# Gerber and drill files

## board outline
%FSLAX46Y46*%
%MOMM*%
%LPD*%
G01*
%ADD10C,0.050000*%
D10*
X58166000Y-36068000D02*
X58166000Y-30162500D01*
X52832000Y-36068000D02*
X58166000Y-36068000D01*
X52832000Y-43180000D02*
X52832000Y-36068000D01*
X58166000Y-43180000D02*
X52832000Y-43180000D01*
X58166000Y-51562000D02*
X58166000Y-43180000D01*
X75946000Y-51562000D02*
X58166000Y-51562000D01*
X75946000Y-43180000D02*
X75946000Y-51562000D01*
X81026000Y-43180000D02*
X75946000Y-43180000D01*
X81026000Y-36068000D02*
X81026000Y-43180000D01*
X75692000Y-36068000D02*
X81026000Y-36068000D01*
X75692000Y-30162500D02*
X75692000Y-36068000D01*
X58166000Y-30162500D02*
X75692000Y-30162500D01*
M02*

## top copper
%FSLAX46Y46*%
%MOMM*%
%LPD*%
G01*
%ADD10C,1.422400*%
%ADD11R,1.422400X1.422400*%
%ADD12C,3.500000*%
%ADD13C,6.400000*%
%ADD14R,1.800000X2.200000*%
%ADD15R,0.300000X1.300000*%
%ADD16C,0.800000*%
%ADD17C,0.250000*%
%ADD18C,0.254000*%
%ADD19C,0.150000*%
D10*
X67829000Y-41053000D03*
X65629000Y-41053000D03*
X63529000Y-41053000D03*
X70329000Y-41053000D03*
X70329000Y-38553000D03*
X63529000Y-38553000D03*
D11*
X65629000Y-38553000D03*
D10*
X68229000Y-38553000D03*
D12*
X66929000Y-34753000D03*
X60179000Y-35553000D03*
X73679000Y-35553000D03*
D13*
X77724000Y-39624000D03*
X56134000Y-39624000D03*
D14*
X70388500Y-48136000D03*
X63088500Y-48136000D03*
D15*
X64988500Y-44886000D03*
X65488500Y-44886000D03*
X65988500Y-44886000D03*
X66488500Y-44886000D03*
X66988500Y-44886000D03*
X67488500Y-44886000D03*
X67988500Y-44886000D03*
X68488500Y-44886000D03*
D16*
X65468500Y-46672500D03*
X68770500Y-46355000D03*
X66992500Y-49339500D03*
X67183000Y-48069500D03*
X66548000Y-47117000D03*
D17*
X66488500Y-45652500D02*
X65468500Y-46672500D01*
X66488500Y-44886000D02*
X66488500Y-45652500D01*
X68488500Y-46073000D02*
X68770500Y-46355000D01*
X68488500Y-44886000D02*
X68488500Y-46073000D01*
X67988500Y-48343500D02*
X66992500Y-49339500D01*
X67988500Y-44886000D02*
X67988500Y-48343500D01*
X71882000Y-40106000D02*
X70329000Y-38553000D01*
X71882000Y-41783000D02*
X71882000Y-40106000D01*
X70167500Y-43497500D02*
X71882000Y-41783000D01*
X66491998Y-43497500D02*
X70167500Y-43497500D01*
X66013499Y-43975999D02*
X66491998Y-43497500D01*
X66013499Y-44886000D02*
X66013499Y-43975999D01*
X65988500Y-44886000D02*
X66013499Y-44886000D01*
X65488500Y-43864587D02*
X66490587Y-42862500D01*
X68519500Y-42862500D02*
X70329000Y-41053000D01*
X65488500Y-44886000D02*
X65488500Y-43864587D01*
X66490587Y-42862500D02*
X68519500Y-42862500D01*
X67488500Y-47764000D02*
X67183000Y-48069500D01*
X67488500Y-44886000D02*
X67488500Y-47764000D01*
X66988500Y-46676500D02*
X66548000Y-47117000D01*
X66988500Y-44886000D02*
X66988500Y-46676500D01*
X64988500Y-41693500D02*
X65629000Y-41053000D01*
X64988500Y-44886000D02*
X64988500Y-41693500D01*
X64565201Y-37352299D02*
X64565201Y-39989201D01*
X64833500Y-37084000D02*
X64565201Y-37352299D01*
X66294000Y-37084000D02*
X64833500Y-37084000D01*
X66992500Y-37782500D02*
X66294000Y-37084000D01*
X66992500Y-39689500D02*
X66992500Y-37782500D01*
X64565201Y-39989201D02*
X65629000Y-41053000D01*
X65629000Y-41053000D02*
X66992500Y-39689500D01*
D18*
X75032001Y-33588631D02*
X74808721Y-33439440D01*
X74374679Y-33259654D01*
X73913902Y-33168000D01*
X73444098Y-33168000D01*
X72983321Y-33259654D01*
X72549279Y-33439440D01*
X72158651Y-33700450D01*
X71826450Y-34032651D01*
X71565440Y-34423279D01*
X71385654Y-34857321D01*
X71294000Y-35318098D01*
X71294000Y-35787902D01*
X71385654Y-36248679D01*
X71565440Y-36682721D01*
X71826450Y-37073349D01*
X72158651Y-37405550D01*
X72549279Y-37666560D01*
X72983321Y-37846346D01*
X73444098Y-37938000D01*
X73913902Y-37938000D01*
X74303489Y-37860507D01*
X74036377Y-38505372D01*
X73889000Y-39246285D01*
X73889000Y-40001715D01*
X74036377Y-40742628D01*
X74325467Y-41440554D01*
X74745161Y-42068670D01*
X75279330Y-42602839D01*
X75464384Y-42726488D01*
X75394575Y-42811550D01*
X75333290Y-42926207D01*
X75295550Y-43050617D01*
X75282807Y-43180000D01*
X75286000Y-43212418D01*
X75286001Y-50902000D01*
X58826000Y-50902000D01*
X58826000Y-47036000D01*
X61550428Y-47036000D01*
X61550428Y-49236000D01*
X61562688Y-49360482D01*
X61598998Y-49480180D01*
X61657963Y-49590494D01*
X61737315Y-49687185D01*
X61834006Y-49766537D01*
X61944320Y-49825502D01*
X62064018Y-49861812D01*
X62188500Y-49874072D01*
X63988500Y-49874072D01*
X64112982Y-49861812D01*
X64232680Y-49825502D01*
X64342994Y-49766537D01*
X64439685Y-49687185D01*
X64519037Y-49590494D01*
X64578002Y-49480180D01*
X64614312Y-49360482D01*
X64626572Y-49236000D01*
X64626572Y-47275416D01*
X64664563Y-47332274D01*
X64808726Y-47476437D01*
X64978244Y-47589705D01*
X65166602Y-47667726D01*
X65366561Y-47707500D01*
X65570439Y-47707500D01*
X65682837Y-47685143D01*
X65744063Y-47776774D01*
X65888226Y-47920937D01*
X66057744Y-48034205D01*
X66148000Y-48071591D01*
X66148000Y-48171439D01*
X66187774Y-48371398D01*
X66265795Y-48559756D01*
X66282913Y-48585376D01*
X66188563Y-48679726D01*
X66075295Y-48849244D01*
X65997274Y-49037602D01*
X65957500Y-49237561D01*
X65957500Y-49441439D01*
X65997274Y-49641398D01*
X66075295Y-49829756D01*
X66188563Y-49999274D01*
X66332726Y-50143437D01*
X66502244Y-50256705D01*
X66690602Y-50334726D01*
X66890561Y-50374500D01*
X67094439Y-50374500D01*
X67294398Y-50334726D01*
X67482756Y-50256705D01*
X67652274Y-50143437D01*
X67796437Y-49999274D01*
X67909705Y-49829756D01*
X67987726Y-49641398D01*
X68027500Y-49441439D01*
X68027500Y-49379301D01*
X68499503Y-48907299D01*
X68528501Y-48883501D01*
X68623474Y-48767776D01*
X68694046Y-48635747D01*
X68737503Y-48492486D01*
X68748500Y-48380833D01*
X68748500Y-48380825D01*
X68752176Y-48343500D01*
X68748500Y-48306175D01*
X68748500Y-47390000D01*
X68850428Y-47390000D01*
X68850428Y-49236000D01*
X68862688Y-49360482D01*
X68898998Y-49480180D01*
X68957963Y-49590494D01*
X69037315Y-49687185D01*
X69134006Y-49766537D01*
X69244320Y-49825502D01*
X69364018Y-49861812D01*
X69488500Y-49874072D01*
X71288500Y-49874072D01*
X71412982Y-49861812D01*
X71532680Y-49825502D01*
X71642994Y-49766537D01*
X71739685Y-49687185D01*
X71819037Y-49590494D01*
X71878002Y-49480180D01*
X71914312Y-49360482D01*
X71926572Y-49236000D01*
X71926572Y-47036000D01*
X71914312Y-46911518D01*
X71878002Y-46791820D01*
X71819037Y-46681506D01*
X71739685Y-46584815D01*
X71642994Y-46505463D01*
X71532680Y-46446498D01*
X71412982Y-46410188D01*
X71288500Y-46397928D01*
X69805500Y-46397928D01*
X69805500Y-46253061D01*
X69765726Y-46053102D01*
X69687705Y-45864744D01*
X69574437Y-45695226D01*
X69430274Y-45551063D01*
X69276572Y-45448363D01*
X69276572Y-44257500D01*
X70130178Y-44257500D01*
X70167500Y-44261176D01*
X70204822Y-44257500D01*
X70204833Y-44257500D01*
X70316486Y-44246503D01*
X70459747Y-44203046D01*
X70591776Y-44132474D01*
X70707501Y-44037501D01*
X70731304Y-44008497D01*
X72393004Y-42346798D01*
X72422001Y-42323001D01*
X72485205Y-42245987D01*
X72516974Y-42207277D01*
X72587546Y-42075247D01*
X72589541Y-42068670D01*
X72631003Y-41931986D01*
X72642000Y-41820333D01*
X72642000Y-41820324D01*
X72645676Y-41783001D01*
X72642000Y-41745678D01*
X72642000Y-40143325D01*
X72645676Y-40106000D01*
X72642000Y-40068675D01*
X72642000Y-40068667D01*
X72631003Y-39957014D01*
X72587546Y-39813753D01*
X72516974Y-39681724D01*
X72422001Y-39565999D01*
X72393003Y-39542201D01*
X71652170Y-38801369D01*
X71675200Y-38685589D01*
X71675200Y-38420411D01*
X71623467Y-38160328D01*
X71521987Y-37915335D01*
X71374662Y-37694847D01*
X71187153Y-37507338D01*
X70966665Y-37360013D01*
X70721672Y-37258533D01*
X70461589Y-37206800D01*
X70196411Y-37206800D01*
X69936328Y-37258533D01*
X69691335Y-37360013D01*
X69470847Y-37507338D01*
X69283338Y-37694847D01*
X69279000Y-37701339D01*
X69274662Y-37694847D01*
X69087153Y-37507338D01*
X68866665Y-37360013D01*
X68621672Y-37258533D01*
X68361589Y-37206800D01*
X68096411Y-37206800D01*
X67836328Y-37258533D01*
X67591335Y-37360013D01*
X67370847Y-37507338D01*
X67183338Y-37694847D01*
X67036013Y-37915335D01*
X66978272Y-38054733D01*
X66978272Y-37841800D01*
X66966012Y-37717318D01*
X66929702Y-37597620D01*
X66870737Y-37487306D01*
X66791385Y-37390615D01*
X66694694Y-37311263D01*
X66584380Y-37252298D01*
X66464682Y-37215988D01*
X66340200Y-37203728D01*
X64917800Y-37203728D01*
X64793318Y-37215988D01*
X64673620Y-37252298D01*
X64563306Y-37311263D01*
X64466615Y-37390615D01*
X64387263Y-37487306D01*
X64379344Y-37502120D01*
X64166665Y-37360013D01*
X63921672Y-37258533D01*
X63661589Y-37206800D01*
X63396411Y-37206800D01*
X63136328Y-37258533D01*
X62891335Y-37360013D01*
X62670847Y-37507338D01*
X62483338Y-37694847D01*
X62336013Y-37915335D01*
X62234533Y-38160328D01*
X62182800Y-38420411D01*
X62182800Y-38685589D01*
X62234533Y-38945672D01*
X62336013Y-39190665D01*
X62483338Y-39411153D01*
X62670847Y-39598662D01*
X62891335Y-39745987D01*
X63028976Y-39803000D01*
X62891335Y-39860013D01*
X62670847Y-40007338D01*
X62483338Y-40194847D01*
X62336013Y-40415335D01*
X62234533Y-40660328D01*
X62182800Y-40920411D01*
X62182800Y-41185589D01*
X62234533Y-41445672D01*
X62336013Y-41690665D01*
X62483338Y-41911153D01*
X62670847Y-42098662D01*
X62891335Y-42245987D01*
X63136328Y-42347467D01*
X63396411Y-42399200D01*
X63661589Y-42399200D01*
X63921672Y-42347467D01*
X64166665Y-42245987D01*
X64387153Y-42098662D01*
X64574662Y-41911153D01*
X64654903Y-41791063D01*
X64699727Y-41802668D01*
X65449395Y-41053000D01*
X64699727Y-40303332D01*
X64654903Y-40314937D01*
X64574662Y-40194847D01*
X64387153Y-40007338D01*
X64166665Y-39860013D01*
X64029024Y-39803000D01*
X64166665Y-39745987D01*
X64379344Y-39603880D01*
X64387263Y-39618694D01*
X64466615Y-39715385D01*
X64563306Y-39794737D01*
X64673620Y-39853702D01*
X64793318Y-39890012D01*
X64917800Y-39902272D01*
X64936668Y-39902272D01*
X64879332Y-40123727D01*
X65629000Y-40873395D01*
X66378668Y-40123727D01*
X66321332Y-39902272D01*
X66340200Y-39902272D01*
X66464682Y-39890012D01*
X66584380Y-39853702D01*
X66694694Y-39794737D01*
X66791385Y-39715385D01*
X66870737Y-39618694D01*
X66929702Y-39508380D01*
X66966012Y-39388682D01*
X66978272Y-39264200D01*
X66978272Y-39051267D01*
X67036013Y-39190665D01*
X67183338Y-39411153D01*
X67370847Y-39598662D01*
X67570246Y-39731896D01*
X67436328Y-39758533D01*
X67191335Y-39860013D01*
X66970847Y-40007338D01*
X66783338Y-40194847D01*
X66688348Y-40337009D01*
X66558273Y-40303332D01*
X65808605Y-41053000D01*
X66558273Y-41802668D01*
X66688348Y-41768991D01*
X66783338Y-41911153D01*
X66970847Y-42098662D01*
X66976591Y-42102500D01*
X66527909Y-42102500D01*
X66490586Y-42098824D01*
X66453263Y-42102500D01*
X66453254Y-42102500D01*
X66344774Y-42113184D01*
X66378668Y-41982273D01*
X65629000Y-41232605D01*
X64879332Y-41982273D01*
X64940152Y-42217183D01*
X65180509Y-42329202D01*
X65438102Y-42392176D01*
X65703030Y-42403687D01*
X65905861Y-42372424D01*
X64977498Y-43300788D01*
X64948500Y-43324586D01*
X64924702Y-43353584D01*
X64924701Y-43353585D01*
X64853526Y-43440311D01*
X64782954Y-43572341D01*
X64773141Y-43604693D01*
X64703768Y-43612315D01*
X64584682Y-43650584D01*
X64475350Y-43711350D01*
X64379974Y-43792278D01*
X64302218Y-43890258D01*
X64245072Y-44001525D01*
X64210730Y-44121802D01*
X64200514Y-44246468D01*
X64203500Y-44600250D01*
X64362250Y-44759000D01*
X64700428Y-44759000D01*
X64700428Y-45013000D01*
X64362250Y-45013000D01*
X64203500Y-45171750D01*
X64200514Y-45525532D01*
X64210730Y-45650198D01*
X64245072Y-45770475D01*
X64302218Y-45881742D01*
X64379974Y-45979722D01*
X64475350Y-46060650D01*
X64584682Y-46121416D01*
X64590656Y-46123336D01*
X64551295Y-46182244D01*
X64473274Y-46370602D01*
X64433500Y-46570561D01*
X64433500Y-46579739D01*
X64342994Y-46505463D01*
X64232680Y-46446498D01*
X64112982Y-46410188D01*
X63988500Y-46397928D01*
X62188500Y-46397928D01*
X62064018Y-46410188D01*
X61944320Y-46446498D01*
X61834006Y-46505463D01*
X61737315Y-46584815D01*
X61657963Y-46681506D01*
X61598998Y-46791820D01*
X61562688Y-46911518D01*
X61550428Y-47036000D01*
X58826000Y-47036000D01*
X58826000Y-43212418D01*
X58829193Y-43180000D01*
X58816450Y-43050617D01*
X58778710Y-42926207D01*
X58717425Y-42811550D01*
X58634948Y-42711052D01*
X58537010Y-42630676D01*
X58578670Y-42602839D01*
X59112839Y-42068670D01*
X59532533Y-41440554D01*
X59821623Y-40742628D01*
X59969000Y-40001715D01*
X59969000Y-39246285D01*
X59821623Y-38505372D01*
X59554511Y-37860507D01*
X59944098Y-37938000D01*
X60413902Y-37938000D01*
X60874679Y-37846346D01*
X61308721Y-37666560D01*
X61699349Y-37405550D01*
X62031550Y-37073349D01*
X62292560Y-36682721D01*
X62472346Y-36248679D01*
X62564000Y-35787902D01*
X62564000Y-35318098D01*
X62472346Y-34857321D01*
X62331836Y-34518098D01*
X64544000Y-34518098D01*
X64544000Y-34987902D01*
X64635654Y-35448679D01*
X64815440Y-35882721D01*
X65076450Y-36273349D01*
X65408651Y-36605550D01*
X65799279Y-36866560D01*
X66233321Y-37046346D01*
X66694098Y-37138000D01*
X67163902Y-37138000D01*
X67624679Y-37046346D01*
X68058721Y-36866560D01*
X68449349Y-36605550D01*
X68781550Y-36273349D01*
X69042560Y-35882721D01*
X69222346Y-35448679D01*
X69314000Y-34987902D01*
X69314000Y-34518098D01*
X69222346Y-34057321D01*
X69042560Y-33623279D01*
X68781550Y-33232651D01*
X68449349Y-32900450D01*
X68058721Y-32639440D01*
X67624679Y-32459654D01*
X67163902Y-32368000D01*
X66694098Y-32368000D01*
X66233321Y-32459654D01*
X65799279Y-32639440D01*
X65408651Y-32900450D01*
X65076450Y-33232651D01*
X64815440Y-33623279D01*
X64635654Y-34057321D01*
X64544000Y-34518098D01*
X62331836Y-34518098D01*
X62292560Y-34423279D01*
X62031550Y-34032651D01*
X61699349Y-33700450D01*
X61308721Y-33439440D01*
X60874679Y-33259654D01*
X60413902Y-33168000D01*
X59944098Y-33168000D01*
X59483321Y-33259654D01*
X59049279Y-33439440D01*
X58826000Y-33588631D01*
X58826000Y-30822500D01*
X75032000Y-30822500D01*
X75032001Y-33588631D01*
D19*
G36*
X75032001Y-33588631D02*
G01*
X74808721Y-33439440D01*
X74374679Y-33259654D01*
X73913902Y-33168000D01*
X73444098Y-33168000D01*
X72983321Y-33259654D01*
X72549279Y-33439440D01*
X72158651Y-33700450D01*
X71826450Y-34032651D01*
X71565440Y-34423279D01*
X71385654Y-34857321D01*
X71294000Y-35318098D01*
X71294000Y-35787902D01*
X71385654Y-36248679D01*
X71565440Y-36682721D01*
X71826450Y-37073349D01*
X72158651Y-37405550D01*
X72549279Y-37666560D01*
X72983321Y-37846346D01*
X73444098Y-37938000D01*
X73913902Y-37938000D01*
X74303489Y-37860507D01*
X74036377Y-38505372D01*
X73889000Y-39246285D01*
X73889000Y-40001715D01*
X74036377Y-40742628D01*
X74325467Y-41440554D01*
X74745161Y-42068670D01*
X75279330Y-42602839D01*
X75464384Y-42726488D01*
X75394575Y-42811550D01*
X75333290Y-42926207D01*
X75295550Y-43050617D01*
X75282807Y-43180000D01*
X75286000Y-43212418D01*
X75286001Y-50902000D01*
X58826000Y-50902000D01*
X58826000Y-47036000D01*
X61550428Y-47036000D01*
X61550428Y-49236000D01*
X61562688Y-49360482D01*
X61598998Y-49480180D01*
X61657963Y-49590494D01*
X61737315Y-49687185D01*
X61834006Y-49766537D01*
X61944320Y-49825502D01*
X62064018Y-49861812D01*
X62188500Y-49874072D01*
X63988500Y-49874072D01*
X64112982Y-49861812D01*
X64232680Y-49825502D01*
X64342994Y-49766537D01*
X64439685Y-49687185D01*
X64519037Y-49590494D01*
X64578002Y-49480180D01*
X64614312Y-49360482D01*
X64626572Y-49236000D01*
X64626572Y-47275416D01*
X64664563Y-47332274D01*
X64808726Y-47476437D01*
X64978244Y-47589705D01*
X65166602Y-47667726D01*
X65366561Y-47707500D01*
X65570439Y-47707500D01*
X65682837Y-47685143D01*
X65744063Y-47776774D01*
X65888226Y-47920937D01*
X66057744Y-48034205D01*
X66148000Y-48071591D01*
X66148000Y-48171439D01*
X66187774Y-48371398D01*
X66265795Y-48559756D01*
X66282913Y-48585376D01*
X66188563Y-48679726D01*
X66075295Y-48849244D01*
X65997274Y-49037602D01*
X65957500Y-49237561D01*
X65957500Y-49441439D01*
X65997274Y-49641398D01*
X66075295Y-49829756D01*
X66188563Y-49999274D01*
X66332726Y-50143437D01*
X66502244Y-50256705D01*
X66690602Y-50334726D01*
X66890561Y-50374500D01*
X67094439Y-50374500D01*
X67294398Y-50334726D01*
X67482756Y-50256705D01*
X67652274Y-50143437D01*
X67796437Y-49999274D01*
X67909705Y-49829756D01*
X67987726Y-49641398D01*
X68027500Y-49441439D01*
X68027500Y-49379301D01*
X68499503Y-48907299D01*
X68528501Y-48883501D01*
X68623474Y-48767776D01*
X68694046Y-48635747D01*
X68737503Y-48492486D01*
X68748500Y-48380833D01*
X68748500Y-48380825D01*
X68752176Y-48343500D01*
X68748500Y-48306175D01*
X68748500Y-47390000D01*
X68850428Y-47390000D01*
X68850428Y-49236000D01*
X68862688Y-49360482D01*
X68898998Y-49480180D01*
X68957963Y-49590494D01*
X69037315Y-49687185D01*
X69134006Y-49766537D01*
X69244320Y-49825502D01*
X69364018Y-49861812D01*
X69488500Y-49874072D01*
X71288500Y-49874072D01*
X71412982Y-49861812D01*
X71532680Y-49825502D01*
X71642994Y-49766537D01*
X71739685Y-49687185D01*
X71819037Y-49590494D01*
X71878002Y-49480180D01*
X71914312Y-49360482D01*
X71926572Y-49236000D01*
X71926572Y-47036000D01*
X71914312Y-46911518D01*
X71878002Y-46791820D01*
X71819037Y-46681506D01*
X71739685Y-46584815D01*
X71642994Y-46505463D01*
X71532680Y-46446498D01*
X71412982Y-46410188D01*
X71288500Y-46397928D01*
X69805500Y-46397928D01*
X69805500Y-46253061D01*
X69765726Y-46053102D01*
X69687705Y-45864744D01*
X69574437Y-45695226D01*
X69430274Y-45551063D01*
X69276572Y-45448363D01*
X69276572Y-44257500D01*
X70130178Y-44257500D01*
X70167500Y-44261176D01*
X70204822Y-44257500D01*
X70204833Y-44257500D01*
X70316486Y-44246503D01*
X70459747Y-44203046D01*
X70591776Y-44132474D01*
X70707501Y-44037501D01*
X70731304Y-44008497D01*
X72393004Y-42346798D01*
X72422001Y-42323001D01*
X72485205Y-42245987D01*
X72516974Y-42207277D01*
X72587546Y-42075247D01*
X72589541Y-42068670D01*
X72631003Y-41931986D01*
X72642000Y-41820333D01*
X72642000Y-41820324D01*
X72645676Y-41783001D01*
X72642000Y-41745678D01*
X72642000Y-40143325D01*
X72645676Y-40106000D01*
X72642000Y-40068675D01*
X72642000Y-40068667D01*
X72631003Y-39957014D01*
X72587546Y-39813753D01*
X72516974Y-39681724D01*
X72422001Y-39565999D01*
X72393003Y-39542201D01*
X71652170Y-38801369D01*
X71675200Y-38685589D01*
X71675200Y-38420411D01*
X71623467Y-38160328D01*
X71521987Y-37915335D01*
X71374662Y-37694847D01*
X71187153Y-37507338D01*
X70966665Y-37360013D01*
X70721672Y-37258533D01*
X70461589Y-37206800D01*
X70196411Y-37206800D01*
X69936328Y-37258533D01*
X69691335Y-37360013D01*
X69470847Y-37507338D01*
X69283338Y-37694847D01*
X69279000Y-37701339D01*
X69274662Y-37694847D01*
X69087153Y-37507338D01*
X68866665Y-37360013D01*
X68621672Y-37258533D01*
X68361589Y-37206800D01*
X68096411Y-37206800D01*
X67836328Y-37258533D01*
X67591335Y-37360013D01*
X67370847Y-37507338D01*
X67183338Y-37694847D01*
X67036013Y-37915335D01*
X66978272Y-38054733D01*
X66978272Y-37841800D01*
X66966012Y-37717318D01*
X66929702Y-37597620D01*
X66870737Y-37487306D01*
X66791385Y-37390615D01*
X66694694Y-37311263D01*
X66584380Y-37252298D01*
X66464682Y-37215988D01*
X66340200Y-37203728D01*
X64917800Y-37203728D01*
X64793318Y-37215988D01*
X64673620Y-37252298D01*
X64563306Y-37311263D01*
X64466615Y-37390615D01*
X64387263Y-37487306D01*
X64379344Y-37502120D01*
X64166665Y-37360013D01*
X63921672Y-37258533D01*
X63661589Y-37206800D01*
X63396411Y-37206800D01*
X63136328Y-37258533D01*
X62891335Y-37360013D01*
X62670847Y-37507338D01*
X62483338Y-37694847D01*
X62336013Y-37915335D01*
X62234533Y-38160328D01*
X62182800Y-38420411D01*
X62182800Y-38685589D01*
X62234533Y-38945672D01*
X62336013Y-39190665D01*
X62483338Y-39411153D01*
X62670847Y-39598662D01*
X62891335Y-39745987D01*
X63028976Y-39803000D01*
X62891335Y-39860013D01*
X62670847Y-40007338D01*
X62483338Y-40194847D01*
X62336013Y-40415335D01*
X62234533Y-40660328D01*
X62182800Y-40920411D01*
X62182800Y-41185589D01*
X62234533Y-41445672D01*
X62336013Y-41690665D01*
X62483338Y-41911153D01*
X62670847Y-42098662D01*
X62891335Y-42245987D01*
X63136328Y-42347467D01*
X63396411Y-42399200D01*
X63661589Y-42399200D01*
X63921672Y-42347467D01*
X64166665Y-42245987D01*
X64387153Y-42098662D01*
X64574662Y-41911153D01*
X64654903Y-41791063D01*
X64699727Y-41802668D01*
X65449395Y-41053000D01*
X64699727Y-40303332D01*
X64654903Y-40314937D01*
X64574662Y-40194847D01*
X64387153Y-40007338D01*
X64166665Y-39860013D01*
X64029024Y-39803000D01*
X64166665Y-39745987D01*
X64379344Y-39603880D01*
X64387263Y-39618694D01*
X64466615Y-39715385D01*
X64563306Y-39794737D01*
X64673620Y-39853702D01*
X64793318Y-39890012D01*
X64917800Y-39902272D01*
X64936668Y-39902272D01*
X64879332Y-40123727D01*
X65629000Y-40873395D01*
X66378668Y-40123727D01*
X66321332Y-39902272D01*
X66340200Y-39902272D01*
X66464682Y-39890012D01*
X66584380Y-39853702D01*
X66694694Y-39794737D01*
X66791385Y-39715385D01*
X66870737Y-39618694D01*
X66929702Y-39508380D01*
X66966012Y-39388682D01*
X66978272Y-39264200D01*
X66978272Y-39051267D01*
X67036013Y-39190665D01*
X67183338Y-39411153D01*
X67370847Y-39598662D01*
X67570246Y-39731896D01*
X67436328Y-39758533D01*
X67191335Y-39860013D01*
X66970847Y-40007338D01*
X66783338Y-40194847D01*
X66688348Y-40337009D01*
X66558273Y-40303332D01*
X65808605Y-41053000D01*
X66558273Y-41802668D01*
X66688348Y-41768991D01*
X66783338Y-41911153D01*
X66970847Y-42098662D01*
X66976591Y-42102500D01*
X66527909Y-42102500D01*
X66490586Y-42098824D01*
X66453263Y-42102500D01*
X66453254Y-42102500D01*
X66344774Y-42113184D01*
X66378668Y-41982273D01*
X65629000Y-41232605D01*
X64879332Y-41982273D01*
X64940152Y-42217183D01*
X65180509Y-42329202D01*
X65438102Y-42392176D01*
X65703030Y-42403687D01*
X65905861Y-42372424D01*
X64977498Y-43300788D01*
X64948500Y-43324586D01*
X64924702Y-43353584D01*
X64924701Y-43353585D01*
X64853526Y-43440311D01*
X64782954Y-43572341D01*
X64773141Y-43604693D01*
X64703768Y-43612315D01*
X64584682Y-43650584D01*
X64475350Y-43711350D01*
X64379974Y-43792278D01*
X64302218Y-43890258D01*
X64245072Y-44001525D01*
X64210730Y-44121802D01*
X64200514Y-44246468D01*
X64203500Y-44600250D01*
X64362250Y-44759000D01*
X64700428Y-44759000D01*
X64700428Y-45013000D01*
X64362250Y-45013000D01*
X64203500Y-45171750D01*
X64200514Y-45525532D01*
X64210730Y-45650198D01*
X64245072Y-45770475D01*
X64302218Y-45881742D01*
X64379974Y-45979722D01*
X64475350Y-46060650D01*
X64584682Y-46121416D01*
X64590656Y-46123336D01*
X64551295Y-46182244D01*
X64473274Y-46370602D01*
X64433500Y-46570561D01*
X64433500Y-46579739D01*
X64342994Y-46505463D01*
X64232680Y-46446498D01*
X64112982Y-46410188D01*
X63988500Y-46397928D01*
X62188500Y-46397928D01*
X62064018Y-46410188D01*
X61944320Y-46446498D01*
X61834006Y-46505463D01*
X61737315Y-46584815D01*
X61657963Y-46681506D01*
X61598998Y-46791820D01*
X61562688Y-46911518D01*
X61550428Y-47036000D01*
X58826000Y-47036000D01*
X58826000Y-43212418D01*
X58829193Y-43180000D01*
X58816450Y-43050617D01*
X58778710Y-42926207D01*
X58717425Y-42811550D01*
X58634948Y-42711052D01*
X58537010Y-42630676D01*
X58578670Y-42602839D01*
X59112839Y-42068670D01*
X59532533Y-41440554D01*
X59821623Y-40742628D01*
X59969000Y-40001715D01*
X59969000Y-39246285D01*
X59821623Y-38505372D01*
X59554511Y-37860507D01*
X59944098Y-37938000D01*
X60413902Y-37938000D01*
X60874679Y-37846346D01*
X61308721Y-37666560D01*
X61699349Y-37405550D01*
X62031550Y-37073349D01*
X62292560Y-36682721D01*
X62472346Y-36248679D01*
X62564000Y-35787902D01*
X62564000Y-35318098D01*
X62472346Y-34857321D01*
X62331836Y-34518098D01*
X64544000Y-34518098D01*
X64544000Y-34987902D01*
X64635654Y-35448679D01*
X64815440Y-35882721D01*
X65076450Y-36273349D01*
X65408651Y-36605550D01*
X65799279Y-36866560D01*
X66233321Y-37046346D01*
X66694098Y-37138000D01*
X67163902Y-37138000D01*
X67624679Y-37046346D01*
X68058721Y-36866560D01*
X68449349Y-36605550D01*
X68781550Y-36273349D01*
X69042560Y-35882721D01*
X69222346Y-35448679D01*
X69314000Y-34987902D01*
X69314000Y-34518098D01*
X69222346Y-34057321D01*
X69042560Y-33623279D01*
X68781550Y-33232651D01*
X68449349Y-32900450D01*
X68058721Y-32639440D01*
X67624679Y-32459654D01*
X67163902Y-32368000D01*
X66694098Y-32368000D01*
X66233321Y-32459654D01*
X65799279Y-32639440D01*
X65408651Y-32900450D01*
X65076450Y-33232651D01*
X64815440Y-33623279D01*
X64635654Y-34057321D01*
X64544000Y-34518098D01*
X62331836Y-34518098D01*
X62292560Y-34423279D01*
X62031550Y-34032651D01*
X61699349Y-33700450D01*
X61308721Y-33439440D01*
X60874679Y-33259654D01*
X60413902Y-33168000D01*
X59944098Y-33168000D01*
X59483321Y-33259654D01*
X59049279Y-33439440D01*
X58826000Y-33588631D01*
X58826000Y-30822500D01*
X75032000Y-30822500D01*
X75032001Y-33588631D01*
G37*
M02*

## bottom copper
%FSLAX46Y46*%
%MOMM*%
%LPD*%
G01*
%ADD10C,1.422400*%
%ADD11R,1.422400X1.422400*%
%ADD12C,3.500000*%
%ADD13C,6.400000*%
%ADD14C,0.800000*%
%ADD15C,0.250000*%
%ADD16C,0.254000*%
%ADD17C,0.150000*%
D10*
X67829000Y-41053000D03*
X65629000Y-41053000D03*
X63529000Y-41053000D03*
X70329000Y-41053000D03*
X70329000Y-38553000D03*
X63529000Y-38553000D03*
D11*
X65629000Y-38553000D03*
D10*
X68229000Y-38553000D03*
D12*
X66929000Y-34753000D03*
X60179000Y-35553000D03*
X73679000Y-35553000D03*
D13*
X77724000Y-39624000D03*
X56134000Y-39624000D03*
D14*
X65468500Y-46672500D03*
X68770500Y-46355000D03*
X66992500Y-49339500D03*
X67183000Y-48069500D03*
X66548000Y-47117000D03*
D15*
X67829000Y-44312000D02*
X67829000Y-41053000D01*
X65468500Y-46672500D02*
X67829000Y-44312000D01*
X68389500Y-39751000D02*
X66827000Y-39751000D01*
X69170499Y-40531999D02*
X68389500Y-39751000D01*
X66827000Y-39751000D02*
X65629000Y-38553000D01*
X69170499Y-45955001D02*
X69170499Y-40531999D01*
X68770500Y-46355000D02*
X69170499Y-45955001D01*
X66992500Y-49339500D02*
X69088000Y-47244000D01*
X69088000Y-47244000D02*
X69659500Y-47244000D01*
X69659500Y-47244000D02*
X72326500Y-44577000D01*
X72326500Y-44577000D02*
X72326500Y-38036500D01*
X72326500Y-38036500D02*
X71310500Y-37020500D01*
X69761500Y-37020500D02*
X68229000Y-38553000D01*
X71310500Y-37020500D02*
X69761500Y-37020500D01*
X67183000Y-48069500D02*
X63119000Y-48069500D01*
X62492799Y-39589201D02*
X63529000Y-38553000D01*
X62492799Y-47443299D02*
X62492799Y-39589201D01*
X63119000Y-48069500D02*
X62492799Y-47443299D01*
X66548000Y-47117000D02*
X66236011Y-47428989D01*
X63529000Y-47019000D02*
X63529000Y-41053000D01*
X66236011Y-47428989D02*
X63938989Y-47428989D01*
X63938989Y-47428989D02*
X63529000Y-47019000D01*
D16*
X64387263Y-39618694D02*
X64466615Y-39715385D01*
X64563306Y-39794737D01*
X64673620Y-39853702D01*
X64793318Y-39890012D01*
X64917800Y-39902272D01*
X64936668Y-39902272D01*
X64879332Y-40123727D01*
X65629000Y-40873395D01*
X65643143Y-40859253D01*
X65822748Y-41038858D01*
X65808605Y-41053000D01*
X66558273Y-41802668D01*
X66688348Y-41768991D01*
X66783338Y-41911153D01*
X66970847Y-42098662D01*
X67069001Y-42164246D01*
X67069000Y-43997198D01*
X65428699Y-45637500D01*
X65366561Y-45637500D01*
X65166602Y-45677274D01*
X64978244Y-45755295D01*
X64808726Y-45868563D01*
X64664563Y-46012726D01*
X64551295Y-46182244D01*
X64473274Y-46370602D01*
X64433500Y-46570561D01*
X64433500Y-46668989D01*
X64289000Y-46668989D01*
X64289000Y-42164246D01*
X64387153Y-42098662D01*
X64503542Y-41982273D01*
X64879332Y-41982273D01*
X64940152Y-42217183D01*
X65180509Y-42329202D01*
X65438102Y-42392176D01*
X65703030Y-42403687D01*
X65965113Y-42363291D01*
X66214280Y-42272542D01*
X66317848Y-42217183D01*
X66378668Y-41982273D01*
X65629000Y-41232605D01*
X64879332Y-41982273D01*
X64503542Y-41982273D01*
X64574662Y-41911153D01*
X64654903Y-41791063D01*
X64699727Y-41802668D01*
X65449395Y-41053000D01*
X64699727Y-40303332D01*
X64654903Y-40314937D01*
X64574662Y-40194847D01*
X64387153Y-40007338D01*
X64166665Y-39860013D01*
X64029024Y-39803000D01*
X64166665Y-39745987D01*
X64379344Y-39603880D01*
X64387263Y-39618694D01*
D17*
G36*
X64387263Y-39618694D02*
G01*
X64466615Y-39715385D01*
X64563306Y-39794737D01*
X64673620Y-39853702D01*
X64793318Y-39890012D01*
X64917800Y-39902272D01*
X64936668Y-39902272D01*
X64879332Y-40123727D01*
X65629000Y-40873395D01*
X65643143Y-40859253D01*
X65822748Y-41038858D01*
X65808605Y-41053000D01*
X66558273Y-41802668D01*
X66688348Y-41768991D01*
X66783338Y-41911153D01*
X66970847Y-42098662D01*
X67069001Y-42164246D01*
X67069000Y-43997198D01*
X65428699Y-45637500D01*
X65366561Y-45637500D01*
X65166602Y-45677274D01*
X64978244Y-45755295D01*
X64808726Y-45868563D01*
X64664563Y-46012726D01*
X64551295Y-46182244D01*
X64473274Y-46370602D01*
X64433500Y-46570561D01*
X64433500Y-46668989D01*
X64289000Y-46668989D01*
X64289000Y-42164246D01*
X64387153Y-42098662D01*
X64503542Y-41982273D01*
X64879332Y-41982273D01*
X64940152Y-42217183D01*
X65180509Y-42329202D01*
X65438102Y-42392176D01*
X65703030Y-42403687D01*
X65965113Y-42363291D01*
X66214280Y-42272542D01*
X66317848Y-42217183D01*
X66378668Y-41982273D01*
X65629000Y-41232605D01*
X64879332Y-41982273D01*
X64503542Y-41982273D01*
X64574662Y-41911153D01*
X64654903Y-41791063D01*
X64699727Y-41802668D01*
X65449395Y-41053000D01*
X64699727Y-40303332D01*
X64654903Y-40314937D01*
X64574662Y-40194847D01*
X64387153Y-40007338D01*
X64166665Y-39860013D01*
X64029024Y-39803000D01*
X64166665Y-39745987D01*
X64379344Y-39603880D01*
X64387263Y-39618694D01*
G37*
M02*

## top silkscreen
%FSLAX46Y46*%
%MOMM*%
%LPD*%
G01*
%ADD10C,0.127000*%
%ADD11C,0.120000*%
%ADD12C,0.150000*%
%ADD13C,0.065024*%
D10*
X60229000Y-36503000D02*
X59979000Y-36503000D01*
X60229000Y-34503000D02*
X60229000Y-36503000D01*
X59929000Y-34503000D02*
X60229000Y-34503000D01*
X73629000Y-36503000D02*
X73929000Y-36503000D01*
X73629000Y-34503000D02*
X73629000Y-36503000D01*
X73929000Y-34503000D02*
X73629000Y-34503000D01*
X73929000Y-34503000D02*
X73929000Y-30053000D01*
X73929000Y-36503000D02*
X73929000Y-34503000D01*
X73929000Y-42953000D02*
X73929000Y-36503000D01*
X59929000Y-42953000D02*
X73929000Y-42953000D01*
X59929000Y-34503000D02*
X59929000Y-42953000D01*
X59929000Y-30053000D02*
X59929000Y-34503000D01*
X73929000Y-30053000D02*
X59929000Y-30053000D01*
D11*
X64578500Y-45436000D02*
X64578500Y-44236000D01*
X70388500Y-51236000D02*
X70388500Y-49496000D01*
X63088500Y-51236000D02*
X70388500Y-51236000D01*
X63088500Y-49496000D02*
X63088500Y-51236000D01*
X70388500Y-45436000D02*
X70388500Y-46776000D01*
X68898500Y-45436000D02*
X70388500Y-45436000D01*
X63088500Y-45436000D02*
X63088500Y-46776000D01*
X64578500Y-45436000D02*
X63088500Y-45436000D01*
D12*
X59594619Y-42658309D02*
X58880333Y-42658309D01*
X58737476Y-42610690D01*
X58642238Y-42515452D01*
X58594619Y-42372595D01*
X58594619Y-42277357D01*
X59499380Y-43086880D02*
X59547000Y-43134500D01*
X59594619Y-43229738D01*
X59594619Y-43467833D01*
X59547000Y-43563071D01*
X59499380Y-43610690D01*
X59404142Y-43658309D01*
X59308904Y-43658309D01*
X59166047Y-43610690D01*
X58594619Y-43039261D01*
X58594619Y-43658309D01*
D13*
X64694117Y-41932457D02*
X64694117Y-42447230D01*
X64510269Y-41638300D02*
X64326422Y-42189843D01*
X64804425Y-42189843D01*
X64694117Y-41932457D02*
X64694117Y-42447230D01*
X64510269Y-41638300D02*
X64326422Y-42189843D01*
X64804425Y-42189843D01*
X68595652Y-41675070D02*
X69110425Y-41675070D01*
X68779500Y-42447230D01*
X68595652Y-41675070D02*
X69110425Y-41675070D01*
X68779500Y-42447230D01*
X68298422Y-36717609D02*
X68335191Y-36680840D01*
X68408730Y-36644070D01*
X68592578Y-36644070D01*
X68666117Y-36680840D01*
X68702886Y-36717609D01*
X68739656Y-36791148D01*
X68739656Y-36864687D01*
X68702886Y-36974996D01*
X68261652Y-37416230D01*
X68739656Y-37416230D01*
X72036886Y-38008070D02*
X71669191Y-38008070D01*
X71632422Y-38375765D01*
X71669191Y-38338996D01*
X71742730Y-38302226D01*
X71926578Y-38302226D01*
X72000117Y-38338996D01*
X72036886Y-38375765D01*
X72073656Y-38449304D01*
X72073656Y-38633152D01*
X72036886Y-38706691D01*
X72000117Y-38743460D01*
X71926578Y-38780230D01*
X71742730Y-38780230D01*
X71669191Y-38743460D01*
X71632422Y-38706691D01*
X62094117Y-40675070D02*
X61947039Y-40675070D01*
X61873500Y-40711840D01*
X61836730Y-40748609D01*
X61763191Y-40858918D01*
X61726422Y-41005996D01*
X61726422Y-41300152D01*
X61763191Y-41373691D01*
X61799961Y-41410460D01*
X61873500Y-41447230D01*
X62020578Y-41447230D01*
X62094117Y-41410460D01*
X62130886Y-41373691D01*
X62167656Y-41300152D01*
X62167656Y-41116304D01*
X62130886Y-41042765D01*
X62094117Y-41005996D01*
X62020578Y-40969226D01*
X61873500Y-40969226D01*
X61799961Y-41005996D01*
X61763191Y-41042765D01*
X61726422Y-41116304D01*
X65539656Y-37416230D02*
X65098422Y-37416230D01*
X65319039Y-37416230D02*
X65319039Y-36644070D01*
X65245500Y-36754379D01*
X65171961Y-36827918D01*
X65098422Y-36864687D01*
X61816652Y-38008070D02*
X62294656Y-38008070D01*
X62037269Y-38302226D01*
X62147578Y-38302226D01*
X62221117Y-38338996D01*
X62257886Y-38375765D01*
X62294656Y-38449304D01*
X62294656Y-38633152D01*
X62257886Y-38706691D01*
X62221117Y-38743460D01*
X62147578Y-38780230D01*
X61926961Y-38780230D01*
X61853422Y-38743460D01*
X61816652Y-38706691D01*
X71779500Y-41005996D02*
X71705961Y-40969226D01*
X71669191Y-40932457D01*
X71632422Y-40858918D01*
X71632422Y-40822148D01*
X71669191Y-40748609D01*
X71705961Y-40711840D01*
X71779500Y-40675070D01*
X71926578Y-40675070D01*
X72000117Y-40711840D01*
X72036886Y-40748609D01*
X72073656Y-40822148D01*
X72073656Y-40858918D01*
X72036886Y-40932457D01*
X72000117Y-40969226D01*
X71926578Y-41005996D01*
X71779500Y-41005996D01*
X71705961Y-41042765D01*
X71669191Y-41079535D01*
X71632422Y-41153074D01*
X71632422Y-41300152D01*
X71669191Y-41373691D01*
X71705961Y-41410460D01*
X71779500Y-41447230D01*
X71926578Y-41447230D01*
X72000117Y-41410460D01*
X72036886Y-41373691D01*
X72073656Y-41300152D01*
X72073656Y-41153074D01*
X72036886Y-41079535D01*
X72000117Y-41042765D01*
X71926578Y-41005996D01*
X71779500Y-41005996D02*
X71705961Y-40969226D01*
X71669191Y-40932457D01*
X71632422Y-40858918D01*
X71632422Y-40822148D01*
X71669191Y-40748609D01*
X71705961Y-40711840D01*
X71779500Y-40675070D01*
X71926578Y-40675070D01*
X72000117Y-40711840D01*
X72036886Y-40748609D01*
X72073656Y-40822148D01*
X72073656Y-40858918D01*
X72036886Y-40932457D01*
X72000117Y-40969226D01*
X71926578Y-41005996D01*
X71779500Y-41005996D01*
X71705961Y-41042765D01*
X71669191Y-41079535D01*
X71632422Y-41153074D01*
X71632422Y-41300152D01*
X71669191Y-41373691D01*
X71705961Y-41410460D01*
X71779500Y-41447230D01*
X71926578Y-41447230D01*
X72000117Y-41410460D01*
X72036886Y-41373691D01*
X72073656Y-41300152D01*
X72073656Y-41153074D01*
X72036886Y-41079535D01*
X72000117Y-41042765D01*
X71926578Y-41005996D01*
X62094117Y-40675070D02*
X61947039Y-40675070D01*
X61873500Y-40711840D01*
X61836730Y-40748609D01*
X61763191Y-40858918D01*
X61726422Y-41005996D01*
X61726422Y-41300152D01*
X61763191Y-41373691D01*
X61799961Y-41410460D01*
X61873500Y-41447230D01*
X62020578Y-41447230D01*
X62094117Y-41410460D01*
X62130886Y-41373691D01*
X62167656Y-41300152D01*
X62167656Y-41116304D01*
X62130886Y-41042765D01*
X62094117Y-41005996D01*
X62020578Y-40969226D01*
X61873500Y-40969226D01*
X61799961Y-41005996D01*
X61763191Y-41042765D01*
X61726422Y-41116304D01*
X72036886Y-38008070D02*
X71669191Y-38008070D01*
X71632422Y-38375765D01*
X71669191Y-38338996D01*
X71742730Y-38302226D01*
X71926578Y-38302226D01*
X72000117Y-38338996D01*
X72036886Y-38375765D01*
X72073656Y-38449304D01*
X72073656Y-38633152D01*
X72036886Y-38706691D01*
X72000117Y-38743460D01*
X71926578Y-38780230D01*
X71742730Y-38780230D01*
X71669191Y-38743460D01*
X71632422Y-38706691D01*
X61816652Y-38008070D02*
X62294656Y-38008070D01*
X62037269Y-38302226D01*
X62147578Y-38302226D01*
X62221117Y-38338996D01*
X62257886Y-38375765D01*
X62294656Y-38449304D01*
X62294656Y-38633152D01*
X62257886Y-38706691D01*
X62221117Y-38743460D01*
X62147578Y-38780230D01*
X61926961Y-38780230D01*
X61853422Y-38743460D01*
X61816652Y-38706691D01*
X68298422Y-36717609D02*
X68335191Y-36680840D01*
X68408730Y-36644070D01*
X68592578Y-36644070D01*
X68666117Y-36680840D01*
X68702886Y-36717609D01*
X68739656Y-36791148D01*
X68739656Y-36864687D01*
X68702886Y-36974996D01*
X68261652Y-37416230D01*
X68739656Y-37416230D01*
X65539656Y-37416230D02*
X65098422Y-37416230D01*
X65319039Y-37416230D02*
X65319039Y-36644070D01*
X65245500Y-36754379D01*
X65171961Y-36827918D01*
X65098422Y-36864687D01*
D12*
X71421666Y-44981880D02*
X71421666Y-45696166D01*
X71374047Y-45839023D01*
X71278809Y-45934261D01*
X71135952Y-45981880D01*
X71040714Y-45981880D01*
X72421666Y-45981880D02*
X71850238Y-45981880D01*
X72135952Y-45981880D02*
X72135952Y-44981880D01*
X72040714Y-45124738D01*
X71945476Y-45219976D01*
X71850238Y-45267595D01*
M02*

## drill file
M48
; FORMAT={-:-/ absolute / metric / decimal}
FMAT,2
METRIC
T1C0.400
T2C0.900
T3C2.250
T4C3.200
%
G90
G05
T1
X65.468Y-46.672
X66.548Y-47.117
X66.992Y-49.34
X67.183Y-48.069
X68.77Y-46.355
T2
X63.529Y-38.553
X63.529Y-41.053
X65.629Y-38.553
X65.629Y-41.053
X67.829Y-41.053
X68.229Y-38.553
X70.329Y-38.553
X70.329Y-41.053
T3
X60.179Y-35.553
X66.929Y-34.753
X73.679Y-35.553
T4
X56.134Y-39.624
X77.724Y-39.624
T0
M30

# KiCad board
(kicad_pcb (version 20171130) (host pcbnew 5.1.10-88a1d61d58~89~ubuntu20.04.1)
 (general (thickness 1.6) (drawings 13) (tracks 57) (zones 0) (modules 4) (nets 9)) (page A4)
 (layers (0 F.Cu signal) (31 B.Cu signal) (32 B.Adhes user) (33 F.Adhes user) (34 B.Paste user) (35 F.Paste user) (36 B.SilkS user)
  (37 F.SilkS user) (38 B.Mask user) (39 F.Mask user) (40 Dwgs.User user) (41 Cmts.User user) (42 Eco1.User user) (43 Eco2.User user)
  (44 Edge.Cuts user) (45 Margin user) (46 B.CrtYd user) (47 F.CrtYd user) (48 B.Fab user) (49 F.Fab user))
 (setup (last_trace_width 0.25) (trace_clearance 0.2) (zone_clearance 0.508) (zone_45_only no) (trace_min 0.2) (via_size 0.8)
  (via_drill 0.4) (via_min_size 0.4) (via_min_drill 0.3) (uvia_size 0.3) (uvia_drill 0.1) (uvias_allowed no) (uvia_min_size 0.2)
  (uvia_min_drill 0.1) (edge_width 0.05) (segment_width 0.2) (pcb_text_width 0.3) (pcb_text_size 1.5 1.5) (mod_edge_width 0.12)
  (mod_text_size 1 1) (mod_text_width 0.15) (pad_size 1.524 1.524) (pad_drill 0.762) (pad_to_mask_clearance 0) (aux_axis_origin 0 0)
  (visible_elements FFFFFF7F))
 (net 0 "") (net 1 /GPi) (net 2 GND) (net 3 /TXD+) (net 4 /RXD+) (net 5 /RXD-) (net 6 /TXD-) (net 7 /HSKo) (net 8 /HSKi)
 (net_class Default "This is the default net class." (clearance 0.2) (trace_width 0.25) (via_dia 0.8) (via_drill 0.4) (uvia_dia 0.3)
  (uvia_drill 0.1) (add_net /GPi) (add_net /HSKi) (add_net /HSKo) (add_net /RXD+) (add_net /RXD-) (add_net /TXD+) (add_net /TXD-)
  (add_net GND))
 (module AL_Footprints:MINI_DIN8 (layer F.Cu) (at 66.929 34.753)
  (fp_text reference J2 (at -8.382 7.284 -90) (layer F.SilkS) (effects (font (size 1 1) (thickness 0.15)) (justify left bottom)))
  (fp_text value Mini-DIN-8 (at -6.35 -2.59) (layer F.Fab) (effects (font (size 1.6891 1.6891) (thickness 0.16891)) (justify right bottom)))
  (fp_line (start -6.7 1.75) (end -6.95 1.75) (layer F.SilkS) (width 0.127))
  (fp_line (start -6.7 -0.25) (end -6.7 1.75) (layer F.SilkS) (width 0.127))
  (fp_line (start -7 -0.25) (end -6.7 -0.25) (layer F.SilkS) (width 0.127))
  (fp_line (start 6.7 1.75) (end 7 1.75) (layer F.SilkS) (width 0.127))
  (fp_line (start 6.7 -0.25) (end 6.7 1.75) (layer F.SilkS) (width 0.127))
  (fp_line (start 7 -0.25) (end 6.7 -0.25) (layer F.SilkS) (width 0.127))
  (fp_line (start 7 -0.25) (end 7 -4.7) (layer F.SilkS) (width 0.127))
  (fp_line (start 7 1.75) (end 7 -0.25) (layer F.SilkS) (width 0.127))
  (fp_line (start 7 8.2) (end 7 1.75) (layer F.SilkS) (width 0.127))
  (fp_line (start -7 8.2) (end 7 8.2) (layer F.SilkS) (width 0.127))
  (fp_line (start -7 -0.25) (end -7 8.2) (layer F.SilkS) (width 0.127))
  (fp_line (start -7 -4.7) (end -7 -0.25) (layer F.SilkS) (width 0.127))
  (fp_line (start 7 -4.7) (end -7 -4.7) (layer F.SilkS) (width 0.127))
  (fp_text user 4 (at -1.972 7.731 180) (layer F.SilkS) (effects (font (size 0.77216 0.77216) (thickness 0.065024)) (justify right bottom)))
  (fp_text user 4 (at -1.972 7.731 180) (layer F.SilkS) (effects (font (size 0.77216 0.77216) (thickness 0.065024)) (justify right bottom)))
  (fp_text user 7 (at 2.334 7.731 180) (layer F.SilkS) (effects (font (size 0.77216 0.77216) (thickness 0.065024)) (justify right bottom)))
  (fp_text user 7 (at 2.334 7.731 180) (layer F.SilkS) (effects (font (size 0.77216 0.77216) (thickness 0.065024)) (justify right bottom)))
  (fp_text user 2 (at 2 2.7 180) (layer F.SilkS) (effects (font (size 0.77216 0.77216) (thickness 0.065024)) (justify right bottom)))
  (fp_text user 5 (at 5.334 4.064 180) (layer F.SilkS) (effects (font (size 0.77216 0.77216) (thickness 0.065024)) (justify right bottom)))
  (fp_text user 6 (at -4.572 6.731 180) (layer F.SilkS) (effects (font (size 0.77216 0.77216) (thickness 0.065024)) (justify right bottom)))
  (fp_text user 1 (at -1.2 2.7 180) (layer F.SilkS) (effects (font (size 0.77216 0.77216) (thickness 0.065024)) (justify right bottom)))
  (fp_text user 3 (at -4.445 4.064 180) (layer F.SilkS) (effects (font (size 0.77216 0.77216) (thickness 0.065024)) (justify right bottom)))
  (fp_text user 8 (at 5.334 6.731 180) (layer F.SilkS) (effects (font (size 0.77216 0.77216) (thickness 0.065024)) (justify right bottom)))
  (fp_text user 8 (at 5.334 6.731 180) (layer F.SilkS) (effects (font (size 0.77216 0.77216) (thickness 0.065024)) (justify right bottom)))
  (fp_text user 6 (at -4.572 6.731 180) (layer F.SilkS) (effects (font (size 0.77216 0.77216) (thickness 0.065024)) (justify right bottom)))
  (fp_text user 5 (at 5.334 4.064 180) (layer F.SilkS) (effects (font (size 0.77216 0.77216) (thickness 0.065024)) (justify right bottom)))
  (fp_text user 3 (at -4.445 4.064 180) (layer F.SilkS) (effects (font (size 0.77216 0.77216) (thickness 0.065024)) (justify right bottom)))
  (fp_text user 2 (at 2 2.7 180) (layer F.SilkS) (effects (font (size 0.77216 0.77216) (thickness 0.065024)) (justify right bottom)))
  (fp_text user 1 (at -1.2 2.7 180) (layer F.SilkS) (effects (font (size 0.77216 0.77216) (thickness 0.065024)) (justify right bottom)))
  (pad 7 thru_hole circle (at 0.9 6.3) (size 1.4224 1.4224) (drill 0.9) (layers *.Cu *.Mask) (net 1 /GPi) (solder_mask_margin 0.0508))
  (pad 4 thru_hole circle (at -1.3 6.3) (size 1.4224 1.4224) (drill 0.9) (layers *.Cu *.Mask) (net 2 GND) (solder_mask_margin 0.0508))
  (pad 6 thru_hole circle (at -3.4 6.3) (size 1.4224 1.4224) (drill 0.9) (layers *.Cu *.Mask) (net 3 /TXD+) (solder_mask_margin 0.0508))
  (pad 8 thru_hole circle (at 3.4 6.3) (size 1.4224 1.4224) (drill 0.9) (layers *.Cu *.Mask) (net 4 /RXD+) (solder_mask_margin 0.0508))
  (pad 5 thru_hole circle (at 3.4 3.8) (size 1.4224 1.4224) (drill 0.9) (layers *.Cu *.Mask) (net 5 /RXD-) (solder_mask_margin 0.0508))
  (pad 3 thru_hole circle (at -3.4 3.8) (size 1.4224 1.4224) (drill 0.9) (layers *.Cu *.Mask) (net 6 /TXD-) (solder_mask_margin 0.0508))
  (pad 1 thru_hole rect (at -1.3 3.8) (size 1.4224 1.4224) (drill 0.9) (layers *.Cu *.Mask) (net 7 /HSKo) (solder_mask_margin 0.0508))
  (pad 2 thru_hole circle (at 1.3 3.8) (size 1.4224 1.4224) (drill 0.9) (layers *.Cu *.Mask) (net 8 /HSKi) (solder_mask_margin 0.0508))
  (pad SH2 thru_hole circle (at 0 0) (size 3.5 3.5) (drill 2.25) (layers *.Cu *.Mask) (solder_mask_margin 0.0508))
  (pad SH3 thru_hole circle (at -6.75 0.8) (size 3.5 3.5) (drill 2.25) (layers *.Cu *.Mask) (solder_mask_margin 0.0508))
  (pad SH1 thru_hole circle (at 6.75 0.8) (size 3.5 3.5) (drill 2.25) (layers *.Cu *.Mask) (solder_mask_margin 0.0508)))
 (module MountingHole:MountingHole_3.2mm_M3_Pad (layer F.Cu) (at 77.724 39.624)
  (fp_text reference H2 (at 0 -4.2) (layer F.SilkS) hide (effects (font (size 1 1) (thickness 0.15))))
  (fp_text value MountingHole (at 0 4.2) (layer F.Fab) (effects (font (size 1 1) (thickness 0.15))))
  (pad 1 thru_hole circle (at 0 0) (size 6.4 6.4) (drill 3.2) (layers *.Cu *.Mask)))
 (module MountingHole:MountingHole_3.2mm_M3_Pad (layer F.Cu) (at 56.134 39.624)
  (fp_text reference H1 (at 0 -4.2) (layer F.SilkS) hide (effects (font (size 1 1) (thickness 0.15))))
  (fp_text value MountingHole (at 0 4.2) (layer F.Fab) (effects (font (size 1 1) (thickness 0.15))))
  (pad 1 thru_hole circle (at 0 0) (size 6.4 6.4) (drill 3.2) (layers *.Cu *.Mask)))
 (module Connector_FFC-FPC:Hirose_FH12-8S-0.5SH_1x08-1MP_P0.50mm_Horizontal (layer F.Cu) (at 66.7385 46.736)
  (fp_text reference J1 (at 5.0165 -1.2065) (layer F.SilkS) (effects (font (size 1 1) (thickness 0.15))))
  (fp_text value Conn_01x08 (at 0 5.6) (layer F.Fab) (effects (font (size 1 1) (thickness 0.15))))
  (fp_line (start -2.16 -1.3) (end -2.16 -2.5) (layer F.SilkS) (width 0.12))
  (fp_line (start 3.65 4.5) (end 3.65 2.76) (layer F.SilkS) (width 0.12))
  (fp_line (start -3.65 4.5) (end 3.65 4.5) (layer F.SilkS) (width 0.12))
  (fp_line (start -3.65 2.76) (end -3.65 4.5) (layer F.SilkS) (width 0.12))
  (fp_line (start 3.65 -1.3) (end 3.65 0.04) (layer F.SilkS) (width 0.12))
  (fp_line (start 2.16 -1.3) (end 3.65 -1.3) (layer F.SilkS) (width 0.12))
  (fp_line (start -3.65 -1.3) (end -3.65 0.04) (layer F.SilkS) (width 0.12))
  (fp_line (start -2.16 -1.3) (end -3.65 -1.3) (layer F.SilkS) (width 0.12))
  (pad MP smd rect (at 3.65 1.4) (size 1.8 2.2) (layers F.Cu F.Paste F.Mask))
  (pad MP smd rect (at -3.65 1.4) (size 1.8 2.2) (layers F.Cu F.Paste F.Mask))
  (pad 1 smd rect (at -1.75 -1.85) (size 0.3 1.3) (layers F.Cu F.Paste F.Mask) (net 2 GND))
  (pad 2 smd rect (at -1.25 -1.85) (size 0.3 1.3) (layers F.Cu F.Paste F.Mask) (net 4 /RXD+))
  (pad 3 smd rect (at -0.75 -1.85) (size 0.3 1.3) (layers F.Cu F.Paste F.Mask) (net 5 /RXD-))
  (pad 4 smd rect (at -0.25 -1.85) (size 0.3 1.3) (layers F.Cu F.Paste F.Mask) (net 1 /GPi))
  (pad 5 smd rect (at 0.25 -1.85) (size 0.3 1.3) (layers F.Cu F.Paste F.Mask) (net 3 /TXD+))
  (pad 6 smd rect (at 0.75 -1.85) (size 0.3 1.3) (layers F.Cu F.Paste F.Mask) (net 6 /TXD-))
  (pad 7 smd rect (at 1.25 -1.85) (size 0.3 1.3) (layers F.Cu F.Paste F.Mask) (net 8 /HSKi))
  (pad 8 smd rect (at 1.75 -1.85) (size 0.3 1.3) (layers F.Cu F.Paste F.Mask) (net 7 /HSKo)))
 (gr_line (start 58.166 36.068) (end 58.166 30.1625) (layer Edge.Cuts) (width 0.05))
 (gr_line (start 52.832 36.068) (end 58.166 36.068) (layer Edge.Cuts) (width 0.05))
 (gr_line (start 52.832 43.18) (end 52.832 36.068) (layer Edge.Cuts) (width 0.05))
 (gr_line (start 58.166 43.18) (end 52.832 43.18) (layer Edge.Cuts) (width 0.05))
 (gr_line (start 58.166 51.562) (end 58.166 43.18) (layer Edge.Cuts) (width 0.05))
 (gr_line (start 75.946 51.562) (end 58.166 51.562) (layer Edge.Cuts) (width 0.05))
 (gr_line (start 75.946 43.18) (end 75.946 51.562) (layer Edge.Cuts) (width 0.05))
 (gr_line (start 81.026 43.18) (end 75.946 43.18) (layer Edge.Cuts) (width 0.05))
 (gr_line (start 81.026 36.068) (end 81.026 43.18) (layer Edge.Cuts) (width 0.05))
 (gr_line (start 75.692 36.068) (end 81.026 36.068) (layer Edge.Cuts) (width 0.05))
 (gr_line (start 75.692 30.1625) (end 75.692 36.068) (layer Edge.Cuts) (width 0.05))
 (gr_line (start 58.166 30.1625) (end 75.692 30.1625) (layer Edge.Cuts) (width 0.05))
 (via (at 65.4685 46.6725) (size 0.8) (drill 0.4) (layers F.Cu B.Cu) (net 1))
 (segment (start 66.4885 45.6525) (end 65.4685 46.6725) (width 0.25) (layer F.Cu) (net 1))
 (segment (start 66.4885 44.886) (end 66.4885 45.6525) (width 0.25) (layer F.Cu) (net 1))
 (segment (start 67.829 44.312) (end 67.829 41.053) (width 0.25) (layer B.Cu) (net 1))
 (segment (start 65.4685 46.6725) (end 67.829 44.312) (width 0.25) (layer B.Cu) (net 1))
 (via (at 68.7705 46.355) (size 0.8) (drill 0.4) (layers F.Cu B.Cu) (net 7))
 (segment (start 68.4885 46.073) (end 68.7705 46.355) (width 0.25) (layer F.Cu) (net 7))
 (segment (start 68.4885 44.886) (end 68.4885 46.073) (width 0.25) (layer F.Cu) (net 7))
 (segment (start 68.3895 39.751) (end 66.827 39.751) (width 0.25) (layer B.Cu) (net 7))
 (segment (start 69.170499 40.531999) (end 68.3895 39.751) (width 0.25) (layer B.Cu) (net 7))
 (segment (start 66.827 39.751) (end 65.629 38.553) (width 0.25) (layer B.Cu) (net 7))
 (segment (start 69.170499 45.955001) (end 69.170499 40.531999) (width 0.25) (layer B.Cu) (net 7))
 (segment (start 68.7705 46.355) (end 69.170499 45.955001) (width 0.25) (layer B.Cu) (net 7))
 (segment (start 67.9885 48.3435) (end 66.9925 49.3395) (width 0.25) (layer F.Cu) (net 8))
 (via (at 66.9925 49.3395) (size 0.8) (drill 0.4) (layers F.Cu B.Cu) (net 8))
 (segment (start 67.9885 44.886) (end 67.9885 48.3435) (width 0.25) (layer F.Cu) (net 8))
 (segment (start 66.9925 49.3395) (end 69.088 47.244) (width 0.25) (layer B.Cu) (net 8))
 (segment (start 69.088 47.244) (end 69.6595 47.244) (width 0.25) (layer B.Cu) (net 8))
 (segment (start 69.6595 47.244) (end 72.3265 44.577) (width 0.25) (layer B.Cu) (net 8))
 (segment (start 72.3265 44.577) (end 72.3265 38.0365) (width 0.25) (layer B.Cu) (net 8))
 (segment (start 72.3265 38.0365) (end 71.3105 37.0205) (width 0.25) (layer B.Cu) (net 8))
 (segment (start 69.7615 37.0205) (end 68.229 38.553) (width 0.25) (layer B.Cu) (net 8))
 (segment (start 71.3105 37.0205) (end 69.7615 37.0205) (width 0.25) (layer B.Cu) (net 8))
 (segment (start 71.882 40.106) (end 70.329 38.553) (width 0.25) (layer F.Cu) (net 5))
 (segment (start 71.882 41.783) (end 71.882 40.106) (width 0.25) (layer F.Cu) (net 5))
 (segment (start 70.1675 43.4975) (end 71.882 41.783) (width 0.25) (layer F.Cu) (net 5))
 (segment (start 66.491998 43.4975) (end 70.1675 43.4975) (width 0.25) (layer F.Cu) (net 5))
 (segment (start 66.013499 43.975999) (end 66.491998 43.4975) (width 0.25) (layer F.Cu) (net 5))
 (segment (start 66.013499 44.886) (end 66.013499 43.975999) (width 0.25) (layer F.Cu) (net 5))
 (segment (start 65.9885 44.886) (end 66.013499 44.886) (width 0.25) (layer F.Cu) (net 5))
 (segment (start 65.4885 43.864587) (end 66.490587 42.8625) (width 0.25) (layer F.Cu) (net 4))
 (segment (start 68.5195 42.8625) (end 70.329 41.053) (width 0.25) (layer F.Cu) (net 4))
 (segment (start 65.4885 44.886) (end 65.4885 43.864587) (width 0.25) (layer F.Cu) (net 4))
 (segment (start 66.490587 42.8625) (end 68.5195 42.8625) (width 0.25) (layer F.Cu) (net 4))
 (segment (start 67.4885 47.764) (end 67.183 48.0695) (width 0.25) (layer F.Cu) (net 6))
 (via (at 67.183 48.0695) (size 0.8) (drill 0.4) (layers F.Cu B.Cu) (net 6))
 (segment (start 67.4885 44.886) (end 67.4885 47.764) (width 0.25) (layer F.Cu) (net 6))
 (segment (start 67.183 48.0695) (end 63.119 48.0695) (width 0.25) (layer B.Cu) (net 6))
 (segment (start 62.492799 39.589201) (end 63.529 38.553) (width 0.25) (layer B.Cu) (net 6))
 (segment (start 62.492799 47.443299) (end 62.492799 39.589201) (width 0.25) (layer B.Cu) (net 6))
 (segment (start 63.119 48.0695) (end 62.492799 47.443299) (width 0.25) (layer B.Cu) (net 6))
 (via (at 66.548 47.117) (size 0.8) (drill 0.4) (layers F.Cu B.Cu) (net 3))
 (segment (start 66.9885 46.6765) (end 66.548 47.117) (width 0.25) (layer F.Cu) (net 3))
 (segment (start 66.9885 44.886) (end 66.9885 46.6765) (width 0.25) (layer F.Cu) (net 3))
 (segment (start 66.548 47.117) (end 66.236011 47.428989) (width 0.25) (layer B.Cu) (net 3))
 (segment (start 63.529 47.019) (end 63.529 41.053) (width 0.25) (layer B.Cu) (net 3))
 (segment (start 66.236011 47.428989) (end 63.938989 47.428989) (width 0.25) (layer B.Cu) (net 3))
 (segment (start 63.938989 47.428989) (end 63.529 47.019) (width 0.25) (layer B.Cu) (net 3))
 (segment (start 64.9885 41.6935) (end 65.629 41.053) (width 0.25) (layer F.Cu) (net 2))
 (segment (start 64.9885 44.886) (end 64.9885 41.6935) (width 0.25) (layer F.Cu) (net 2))
 (segment (start 64.565201 37.352299) (end 64.565201 39.989201) (width 0.25) (layer F.Cu) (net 2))
 (segment (start 64.8335 37.084) (end 64.565201 37.352299) (width 0.25) (layer F.Cu) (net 2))
 (segment (start 66.294 37.084) (end 64.8335 37.084) (width 0.25) (layer F.Cu) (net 2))
 (segment (start 66.9925 37.7825) (end 66.294 37.084) (width 0.25) (layer F.Cu) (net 2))
 (segment (start 66.9925 39.6895) (end 66.9925 37.7825) (width 0.25) (layer F.Cu) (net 2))
 (segment (start 64.565201 39.989201) (end 65.629 41.053) (width 0.25) (layer F.Cu) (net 2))
 (segment (start 65.629 41.053) (end 66.9925 39.6895) (width 0.25) (layer F.Cu) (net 2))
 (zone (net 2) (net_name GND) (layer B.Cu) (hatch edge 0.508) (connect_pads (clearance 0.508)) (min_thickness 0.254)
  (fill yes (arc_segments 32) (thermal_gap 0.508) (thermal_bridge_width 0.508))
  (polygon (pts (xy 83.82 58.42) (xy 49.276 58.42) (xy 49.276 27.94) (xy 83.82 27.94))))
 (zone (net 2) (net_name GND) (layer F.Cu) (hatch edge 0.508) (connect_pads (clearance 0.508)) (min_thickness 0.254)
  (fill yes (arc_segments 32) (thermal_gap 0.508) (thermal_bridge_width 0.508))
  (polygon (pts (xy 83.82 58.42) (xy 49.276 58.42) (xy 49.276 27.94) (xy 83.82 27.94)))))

